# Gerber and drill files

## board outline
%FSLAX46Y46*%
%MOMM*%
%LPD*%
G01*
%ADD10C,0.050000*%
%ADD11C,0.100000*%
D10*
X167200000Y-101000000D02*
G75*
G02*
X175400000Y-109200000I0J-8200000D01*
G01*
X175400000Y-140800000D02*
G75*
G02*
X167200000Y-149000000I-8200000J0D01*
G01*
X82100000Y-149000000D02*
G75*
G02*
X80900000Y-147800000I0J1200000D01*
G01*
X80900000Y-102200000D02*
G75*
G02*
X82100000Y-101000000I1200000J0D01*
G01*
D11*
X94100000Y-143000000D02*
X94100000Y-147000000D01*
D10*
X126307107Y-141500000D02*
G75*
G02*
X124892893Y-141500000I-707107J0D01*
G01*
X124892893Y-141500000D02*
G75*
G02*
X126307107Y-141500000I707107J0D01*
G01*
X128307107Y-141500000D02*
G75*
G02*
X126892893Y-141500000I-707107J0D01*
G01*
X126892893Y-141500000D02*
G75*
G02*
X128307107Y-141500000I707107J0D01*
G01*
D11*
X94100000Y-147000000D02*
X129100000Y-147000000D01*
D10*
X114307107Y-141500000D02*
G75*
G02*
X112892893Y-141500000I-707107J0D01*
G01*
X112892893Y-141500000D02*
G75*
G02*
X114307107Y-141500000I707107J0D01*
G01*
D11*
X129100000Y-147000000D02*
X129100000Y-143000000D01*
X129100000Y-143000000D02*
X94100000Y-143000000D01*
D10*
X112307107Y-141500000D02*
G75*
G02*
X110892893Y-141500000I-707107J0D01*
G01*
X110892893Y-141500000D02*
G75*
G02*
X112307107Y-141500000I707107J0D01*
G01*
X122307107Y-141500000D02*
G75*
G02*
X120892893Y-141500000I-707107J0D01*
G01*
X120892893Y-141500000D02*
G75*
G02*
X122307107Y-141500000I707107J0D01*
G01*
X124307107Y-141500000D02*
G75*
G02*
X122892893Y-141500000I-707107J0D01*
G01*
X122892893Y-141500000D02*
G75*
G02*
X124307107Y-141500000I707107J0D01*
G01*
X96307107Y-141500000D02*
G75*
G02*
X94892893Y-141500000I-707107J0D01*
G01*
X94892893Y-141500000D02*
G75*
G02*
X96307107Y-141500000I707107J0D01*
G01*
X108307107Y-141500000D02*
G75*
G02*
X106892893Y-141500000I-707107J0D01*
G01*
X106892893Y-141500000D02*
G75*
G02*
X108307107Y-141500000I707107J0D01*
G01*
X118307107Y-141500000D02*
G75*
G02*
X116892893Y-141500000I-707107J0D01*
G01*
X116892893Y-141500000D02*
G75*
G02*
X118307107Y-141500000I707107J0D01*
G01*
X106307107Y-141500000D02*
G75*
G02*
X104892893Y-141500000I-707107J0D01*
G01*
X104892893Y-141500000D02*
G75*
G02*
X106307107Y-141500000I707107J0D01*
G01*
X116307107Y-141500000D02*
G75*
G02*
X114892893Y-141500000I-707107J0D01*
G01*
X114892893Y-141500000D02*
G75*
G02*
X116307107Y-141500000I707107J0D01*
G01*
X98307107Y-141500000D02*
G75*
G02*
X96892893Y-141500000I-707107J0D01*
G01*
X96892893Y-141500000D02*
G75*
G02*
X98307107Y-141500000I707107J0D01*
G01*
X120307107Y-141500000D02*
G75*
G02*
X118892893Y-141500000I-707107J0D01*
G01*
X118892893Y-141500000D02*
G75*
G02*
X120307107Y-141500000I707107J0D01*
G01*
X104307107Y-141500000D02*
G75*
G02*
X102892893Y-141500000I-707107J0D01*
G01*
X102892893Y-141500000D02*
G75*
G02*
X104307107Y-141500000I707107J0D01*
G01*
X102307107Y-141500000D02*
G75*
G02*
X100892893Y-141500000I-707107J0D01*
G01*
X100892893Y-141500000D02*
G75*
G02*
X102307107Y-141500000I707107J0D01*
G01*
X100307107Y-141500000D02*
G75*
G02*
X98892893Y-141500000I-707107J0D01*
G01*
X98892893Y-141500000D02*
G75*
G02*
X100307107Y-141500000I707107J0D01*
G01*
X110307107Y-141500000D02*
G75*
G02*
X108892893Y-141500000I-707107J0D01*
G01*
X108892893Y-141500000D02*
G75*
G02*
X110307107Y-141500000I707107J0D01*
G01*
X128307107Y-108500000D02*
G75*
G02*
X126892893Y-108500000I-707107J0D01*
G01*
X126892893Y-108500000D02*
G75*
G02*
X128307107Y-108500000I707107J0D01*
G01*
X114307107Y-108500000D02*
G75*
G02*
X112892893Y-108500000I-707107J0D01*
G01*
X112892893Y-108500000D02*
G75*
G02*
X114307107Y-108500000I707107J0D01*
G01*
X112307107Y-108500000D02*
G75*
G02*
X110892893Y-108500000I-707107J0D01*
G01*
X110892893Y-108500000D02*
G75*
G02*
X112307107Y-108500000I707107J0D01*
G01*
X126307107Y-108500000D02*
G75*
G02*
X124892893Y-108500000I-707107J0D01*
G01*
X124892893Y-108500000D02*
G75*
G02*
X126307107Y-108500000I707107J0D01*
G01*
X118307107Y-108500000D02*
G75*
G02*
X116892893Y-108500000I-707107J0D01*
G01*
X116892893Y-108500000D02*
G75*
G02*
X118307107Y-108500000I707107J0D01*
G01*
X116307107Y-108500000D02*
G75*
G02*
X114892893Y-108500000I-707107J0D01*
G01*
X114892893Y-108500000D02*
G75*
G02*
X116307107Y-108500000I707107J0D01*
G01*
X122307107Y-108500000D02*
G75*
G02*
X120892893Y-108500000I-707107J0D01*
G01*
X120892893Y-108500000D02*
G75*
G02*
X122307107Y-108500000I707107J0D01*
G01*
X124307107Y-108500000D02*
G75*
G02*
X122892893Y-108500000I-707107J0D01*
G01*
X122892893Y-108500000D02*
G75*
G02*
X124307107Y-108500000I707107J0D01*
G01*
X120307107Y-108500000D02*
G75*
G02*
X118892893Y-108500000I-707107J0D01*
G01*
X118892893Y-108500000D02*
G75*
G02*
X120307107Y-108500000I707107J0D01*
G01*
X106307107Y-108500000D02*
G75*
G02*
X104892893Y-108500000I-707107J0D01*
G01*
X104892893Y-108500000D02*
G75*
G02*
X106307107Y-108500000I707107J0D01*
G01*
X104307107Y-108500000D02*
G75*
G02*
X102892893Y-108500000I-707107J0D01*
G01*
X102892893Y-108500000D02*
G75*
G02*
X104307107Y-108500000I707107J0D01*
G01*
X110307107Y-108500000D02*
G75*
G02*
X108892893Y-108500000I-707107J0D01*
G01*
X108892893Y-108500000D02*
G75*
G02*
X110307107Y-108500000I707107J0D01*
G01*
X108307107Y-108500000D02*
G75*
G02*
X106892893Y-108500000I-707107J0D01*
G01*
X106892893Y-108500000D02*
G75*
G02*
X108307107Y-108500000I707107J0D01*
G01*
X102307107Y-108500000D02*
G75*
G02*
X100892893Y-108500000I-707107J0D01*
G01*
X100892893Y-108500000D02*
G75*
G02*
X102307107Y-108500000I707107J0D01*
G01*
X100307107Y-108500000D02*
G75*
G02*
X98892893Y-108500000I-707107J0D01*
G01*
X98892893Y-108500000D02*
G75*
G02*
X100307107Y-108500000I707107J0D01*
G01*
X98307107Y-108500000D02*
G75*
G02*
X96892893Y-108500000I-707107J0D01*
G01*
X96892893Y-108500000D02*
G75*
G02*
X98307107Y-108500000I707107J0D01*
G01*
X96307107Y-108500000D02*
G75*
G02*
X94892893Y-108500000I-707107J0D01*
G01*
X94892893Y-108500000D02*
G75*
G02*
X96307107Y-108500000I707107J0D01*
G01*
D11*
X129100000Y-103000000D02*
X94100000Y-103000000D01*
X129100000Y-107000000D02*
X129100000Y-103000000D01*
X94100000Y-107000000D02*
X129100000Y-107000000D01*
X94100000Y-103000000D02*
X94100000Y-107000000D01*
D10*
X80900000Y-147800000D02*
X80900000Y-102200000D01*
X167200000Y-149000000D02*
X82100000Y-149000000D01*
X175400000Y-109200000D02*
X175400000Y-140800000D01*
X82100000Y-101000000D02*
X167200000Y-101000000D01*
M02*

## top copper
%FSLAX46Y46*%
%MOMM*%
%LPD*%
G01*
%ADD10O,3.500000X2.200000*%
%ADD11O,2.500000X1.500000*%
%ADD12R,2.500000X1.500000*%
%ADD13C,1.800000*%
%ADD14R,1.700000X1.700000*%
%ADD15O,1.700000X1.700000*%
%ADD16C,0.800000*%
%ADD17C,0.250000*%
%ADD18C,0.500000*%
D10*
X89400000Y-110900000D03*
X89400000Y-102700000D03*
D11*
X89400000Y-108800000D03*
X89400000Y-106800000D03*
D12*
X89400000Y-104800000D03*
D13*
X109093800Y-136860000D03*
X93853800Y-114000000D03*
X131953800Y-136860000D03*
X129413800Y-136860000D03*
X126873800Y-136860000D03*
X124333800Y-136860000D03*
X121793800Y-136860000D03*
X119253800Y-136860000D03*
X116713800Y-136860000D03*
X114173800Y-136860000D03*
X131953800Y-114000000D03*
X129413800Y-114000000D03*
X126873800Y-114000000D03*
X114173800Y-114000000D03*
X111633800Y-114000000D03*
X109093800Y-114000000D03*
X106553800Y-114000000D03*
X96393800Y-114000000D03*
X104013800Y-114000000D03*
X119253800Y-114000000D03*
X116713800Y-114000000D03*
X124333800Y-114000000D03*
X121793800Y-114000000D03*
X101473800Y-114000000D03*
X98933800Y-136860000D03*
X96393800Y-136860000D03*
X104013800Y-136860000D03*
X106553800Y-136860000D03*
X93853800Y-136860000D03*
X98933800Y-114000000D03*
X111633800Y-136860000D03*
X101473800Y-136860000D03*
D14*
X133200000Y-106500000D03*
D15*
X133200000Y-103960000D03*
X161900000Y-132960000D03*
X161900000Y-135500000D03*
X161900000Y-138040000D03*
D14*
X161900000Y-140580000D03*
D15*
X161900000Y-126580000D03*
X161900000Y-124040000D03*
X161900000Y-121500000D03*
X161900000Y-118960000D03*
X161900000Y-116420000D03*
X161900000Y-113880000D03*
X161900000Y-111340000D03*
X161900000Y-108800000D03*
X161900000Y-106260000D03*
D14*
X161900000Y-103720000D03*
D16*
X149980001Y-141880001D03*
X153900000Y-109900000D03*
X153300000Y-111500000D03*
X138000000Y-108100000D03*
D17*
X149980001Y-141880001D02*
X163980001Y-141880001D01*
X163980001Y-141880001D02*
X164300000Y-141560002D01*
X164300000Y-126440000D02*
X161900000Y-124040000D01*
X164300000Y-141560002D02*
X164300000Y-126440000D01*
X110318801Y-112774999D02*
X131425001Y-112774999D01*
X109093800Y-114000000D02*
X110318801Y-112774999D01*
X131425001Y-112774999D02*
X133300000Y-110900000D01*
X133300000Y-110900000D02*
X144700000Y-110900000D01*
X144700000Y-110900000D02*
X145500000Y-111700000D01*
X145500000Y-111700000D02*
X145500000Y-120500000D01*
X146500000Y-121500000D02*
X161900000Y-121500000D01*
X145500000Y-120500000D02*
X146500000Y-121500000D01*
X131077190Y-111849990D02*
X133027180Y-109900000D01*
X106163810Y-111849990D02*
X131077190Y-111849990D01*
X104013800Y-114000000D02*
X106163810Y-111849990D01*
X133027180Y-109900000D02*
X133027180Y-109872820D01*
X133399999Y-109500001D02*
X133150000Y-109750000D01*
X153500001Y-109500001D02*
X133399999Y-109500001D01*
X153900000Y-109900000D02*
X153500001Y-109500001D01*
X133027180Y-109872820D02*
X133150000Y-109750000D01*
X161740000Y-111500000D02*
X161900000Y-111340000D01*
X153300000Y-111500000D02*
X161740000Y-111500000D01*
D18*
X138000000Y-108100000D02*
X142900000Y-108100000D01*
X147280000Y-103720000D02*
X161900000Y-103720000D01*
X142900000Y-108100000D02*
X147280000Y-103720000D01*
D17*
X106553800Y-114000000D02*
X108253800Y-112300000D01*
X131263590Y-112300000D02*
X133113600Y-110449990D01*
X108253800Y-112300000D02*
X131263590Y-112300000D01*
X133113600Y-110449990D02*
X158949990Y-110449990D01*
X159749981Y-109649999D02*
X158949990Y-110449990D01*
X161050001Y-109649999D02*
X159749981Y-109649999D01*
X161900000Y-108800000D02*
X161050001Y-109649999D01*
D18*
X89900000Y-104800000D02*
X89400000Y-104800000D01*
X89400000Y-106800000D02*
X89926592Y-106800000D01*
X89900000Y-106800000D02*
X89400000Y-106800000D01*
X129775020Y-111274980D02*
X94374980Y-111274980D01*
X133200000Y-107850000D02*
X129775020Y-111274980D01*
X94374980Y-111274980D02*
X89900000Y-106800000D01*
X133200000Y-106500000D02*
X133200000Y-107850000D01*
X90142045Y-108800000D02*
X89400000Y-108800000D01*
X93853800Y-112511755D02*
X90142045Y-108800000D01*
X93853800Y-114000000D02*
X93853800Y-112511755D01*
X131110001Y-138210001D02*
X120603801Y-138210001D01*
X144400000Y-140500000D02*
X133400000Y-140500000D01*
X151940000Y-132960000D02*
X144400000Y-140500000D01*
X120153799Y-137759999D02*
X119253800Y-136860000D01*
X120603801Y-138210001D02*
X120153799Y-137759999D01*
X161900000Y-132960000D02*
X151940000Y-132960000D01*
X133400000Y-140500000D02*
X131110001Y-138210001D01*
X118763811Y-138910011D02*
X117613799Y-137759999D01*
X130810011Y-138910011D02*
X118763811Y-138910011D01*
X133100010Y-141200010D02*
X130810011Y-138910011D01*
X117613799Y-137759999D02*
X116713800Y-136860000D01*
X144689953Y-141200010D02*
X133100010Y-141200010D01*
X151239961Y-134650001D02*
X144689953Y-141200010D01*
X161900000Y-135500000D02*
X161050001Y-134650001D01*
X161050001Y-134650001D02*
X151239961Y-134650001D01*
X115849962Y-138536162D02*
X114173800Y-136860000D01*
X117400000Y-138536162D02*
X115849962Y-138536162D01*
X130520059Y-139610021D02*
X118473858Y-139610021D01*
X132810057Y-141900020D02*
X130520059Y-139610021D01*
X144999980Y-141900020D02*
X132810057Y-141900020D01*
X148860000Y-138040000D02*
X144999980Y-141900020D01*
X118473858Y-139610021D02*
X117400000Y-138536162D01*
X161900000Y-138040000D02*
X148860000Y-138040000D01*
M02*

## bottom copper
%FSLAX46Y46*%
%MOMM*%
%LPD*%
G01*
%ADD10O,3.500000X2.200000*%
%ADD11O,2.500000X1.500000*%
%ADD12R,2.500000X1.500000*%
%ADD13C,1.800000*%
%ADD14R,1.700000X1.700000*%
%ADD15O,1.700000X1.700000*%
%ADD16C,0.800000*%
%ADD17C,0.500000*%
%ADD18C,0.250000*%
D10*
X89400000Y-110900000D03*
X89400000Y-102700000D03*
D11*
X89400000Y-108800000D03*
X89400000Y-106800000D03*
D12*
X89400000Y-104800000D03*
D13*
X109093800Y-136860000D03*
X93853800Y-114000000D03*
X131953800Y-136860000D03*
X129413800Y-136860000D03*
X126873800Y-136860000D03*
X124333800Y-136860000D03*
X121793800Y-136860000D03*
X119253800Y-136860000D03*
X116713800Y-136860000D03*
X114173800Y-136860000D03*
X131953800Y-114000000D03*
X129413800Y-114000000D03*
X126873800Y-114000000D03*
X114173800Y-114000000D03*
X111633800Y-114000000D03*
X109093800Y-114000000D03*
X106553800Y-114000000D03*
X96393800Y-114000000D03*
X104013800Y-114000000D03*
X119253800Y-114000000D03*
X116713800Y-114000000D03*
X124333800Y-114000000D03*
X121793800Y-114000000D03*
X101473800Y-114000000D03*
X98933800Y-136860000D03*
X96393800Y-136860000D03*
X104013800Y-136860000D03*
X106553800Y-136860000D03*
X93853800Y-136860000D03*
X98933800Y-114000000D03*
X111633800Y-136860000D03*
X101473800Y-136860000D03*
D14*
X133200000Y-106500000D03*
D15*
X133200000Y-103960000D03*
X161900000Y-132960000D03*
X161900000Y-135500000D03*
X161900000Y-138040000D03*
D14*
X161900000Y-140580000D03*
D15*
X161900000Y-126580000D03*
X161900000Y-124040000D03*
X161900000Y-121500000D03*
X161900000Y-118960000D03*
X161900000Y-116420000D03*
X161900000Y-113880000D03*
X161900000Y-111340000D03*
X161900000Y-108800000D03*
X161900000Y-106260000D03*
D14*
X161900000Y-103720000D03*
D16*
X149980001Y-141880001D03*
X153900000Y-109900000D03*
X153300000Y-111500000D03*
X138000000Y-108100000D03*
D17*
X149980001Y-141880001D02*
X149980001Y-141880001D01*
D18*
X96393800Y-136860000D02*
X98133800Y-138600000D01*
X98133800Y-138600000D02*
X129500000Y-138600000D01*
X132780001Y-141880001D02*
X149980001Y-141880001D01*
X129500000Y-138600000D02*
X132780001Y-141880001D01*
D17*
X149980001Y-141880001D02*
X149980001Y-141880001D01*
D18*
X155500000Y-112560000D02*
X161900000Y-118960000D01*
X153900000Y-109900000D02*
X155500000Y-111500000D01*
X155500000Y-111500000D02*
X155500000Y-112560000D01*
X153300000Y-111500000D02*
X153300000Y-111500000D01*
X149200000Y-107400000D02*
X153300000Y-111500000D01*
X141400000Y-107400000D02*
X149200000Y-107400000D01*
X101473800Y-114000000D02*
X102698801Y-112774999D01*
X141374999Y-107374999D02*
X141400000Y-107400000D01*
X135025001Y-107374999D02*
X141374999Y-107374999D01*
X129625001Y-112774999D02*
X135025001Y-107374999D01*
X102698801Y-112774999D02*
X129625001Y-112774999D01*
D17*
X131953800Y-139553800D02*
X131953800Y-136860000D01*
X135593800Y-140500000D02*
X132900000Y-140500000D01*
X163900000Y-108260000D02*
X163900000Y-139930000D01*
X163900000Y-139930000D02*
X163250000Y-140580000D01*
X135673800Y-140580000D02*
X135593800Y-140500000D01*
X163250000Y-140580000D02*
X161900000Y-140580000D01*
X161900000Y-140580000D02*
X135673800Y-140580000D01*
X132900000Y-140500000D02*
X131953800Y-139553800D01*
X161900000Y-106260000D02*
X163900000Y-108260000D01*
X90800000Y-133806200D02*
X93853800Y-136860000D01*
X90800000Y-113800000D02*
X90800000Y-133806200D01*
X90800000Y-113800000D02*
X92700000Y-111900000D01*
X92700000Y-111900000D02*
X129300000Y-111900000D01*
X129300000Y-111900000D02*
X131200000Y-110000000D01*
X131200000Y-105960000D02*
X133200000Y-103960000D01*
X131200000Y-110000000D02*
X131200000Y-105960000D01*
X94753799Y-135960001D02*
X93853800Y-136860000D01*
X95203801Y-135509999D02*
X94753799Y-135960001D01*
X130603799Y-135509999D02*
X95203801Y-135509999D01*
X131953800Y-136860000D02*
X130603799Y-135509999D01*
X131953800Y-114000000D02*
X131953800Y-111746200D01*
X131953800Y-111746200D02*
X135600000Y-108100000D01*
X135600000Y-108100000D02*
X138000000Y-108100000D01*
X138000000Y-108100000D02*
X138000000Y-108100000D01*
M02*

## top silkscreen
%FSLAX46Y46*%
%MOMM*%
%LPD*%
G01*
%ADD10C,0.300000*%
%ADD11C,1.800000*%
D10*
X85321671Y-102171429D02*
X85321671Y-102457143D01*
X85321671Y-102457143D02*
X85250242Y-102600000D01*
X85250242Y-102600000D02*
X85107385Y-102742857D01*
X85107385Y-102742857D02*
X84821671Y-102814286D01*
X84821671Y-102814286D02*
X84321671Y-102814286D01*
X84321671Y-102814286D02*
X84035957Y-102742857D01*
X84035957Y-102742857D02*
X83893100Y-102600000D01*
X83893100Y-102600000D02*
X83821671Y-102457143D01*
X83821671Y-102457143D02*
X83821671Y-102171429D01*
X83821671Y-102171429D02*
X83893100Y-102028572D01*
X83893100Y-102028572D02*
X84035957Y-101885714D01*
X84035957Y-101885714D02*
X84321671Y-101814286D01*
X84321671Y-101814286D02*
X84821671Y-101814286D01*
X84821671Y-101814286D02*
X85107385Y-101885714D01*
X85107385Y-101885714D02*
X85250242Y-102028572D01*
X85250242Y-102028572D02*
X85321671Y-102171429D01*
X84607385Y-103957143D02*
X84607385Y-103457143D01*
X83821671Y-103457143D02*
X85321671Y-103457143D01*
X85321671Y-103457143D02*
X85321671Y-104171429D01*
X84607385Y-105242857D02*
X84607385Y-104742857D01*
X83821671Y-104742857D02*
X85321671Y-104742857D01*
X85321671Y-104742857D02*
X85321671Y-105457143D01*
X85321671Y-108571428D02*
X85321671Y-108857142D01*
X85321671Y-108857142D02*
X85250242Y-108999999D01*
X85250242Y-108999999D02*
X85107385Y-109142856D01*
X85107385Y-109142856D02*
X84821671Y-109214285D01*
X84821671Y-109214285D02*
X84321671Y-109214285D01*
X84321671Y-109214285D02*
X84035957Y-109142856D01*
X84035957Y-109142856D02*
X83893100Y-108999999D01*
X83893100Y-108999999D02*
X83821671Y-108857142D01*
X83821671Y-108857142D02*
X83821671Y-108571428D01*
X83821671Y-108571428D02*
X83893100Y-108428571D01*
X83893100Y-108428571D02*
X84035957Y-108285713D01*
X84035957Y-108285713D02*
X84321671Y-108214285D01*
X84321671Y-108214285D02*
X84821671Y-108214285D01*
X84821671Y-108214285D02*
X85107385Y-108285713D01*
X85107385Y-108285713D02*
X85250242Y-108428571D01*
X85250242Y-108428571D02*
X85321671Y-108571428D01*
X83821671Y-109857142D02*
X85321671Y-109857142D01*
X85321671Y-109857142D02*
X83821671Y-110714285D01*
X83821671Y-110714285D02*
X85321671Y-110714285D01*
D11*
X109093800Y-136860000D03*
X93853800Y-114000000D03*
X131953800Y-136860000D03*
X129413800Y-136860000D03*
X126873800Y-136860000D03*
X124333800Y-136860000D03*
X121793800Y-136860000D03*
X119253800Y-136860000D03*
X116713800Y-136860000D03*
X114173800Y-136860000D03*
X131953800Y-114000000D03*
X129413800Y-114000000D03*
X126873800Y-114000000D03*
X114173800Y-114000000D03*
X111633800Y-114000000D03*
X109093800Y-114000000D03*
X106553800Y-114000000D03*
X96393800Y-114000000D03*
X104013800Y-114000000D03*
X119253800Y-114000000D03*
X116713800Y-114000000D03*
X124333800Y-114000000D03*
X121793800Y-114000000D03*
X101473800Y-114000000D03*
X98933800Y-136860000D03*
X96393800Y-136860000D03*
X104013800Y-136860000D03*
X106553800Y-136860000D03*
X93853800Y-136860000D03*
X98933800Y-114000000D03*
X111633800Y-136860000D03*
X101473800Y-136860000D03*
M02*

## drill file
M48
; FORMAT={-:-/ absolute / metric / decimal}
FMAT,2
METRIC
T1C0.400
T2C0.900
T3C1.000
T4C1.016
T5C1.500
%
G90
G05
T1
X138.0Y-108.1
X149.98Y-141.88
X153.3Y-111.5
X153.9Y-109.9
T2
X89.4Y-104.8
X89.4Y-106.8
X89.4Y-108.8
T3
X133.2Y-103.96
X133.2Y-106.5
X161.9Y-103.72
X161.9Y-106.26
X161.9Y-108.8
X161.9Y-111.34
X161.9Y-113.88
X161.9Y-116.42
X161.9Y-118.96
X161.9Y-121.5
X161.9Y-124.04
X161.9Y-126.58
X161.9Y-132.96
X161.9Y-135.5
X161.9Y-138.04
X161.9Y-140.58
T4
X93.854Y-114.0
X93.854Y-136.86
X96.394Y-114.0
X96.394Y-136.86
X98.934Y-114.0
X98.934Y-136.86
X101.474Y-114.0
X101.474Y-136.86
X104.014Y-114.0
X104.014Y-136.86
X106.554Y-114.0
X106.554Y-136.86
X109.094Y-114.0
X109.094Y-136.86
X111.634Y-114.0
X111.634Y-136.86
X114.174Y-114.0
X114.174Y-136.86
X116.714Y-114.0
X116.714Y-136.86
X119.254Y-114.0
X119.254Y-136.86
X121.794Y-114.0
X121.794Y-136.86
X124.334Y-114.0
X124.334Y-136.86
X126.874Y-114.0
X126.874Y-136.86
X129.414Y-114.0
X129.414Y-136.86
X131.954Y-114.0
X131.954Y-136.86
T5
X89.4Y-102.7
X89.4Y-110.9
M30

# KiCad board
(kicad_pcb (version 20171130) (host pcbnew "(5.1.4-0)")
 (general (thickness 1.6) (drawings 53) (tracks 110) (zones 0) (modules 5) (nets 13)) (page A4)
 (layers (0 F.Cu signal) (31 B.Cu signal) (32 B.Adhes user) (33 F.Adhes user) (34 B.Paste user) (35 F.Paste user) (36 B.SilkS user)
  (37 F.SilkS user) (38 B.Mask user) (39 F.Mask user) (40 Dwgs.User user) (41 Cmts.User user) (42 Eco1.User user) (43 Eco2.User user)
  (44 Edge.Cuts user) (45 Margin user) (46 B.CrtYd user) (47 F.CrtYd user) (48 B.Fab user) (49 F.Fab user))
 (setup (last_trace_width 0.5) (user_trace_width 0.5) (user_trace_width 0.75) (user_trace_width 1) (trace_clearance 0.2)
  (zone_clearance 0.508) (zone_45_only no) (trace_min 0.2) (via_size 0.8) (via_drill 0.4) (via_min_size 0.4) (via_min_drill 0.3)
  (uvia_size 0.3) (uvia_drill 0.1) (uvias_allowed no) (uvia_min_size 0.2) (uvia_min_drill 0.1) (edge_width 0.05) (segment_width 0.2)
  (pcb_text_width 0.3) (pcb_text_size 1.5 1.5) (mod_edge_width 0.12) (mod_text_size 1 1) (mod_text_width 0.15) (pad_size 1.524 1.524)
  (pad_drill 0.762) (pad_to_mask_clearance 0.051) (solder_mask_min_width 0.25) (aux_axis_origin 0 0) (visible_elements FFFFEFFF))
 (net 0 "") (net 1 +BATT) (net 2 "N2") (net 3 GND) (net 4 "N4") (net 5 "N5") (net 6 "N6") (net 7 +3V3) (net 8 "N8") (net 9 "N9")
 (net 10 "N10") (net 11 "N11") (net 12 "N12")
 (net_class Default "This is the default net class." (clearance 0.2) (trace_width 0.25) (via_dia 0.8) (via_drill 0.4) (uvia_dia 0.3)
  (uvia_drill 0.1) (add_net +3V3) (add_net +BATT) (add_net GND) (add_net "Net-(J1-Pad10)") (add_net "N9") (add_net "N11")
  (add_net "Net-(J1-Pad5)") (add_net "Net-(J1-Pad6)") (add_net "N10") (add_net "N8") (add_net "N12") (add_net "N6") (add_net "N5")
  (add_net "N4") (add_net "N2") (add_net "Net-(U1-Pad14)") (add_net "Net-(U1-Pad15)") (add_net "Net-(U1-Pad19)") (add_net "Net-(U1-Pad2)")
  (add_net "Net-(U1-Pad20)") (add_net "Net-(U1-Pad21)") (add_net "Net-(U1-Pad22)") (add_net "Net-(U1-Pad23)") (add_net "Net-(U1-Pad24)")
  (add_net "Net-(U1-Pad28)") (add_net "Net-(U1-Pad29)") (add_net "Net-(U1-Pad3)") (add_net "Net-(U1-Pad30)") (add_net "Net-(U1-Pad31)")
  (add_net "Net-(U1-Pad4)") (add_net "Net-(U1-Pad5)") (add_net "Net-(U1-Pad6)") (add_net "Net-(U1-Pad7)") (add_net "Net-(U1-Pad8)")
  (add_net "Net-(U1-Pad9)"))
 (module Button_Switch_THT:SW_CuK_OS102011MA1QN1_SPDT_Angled (layer F.Cu) (at 89.4 104.8 270)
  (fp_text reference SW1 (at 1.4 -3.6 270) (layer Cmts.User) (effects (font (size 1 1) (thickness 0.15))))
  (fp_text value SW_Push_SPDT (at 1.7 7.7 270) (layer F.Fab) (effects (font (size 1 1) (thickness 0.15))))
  (pad "" thru_hole oval (at 6.1 0 270) (size 2.2 3.5) (drill 1.5) (layers *.Cu *.Mask))
  (pad "" thru_hole oval (at -2.1 0 270) (size 2.2 3.5) (drill 1.5) (layers *.Cu *.Mask))
  (pad 3 thru_hole oval (at 4 0 270) (size 1.5 2.5) (drill 0.9) (layers *.Cu *.Mask) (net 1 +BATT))
  (pad 2 thru_hole oval (at 2 0 270) (size 1.5 2.5) (drill 0.9) (layers *.Cu *.Mask) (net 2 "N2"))
  (pad 1 thru_hole rect (at 0 0 270) (size 1.5 2.5) (drill 0.9) (layers *.Cu *.Mask)))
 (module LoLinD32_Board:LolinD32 (layer F.Cu) (at 107.9 125.7094 270)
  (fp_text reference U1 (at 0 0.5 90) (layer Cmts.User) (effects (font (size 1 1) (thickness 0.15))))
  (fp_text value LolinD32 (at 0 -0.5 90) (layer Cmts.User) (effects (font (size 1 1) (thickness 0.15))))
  (pad 23 thru_hole circle (at 11.1506 -1.1938 270) (size 1.8 1.8) (drill 1.016) (layers *.Cu *.Mask F.SilkS))
  (pad 16 thru_hole circle (at -11.7094 14.0462 270) (size 1.8 1.8) (drill 1.016) (layers *.Cu *.Mask F.SilkS) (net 1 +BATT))
  (pad 32 thru_hole circle (at 11.1506 -24.0538 270) (size 1.8 1.8) (drill 1.016) (layers *.Cu *.Mask F.SilkS) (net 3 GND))
  (pad 31 thru_hole circle (at 11.1506 -21.5138 270) (size 1.8 1.8) (drill 1.016) (layers *.Cu *.Mask F.SilkS))
  (pad 30 thru_hole circle (at 11.1506 -18.9738 270) (size 1.8 1.8) (drill 1.016) (layers *.Cu *.Mask F.SilkS))
  (pad 29 thru_hole circle (at 11.1506 -16.4338 270) (size 1.8 1.8) (drill 1.016) (layers *.Cu *.Mask F.SilkS))
  (pad 28 thru_hole circle (at 11.1506 -13.8938 270) (size 1.8 1.8) (drill 1.016) (layers *.Cu *.Mask F.SilkS))
  (pad 27 thru_hole circle (at 11.1506 -11.3538 270) (size 1.8 1.8) (drill 1.016) (layers *.Cu *.Mask F.SilkS) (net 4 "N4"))
  (pad 26 thru_hole circle (at 11.1506 -8.8138 270) (size 1.8 1.8) (drill 1.016) (layers *.Cu *.Mask F.SilkS) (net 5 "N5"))
  (pad 25 thru_hole circle (at 11.1506 -6.2738 270) (size 1.8 1.8) (drill 1.016) (layers *.Cu *.Mask F.SilkS) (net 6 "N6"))
  (pad 1 thru_hole circle (at -11.7094 -24.0538 270) (size 1.8 1.8) (drill 1.016) (layers *.Cu *.Mask F.SilkS) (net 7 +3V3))
  (pad 2 thru_hole circle (at -11.7094 -21.5138 270) (size 1.8 1.8) (drill 1.016) (layers *.Cu *.Mask F.SilkS))
  (pad 3 thru_hole circle (at -11.7094 -18.9738 270) (size 1.8 1.8) (drill 1.016) (layers *.Cu *.Mask F.SilkS))
  (pad 8 thru_hole circle (at -11.7094 -6.2738 270) (size 1.8 1.8) (drill 1.016) (layers *.Cu *.Mask F.SilkS))
  (pad 9 thru_hole circle (at -11.7094 -3.7338 270) (size 1.8 1.8) (drill 1.016) (layers *.Cu *.Mask F.SilkS))
  (pad 10 thru_hole circle (at -11.7094 -1.1938 270) (size 1.8 1.8) (drill 1.016) (layers *.Cu *.Mask F.SilkS) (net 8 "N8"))
  (pad 11 thru_hole circle (at -11.7094 1.3462 270) (size 1.8 1.8) (drill 1.016) (layers *.Cu *.Mask F.SilkS) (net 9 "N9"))
  (pad 15 thru_hole circle (at -11.7094 11.5062 270) (size 1.8 1.8) (drill 1.016) (layers *.Cu *.Mask F.SilkS))
  (pad 12 thru_hole circle (at -11.7094 3.8862 270) (size 1.8 1.8) (drill 1.016) (layers *.Cu *.Mask F.SilkS) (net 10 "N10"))
  (pad 6 thru_hole circle (at -11.7094 -11.3538 270) (size 1.8 1.8) (drill 1.016) (layers *.Cu *.Mask F.SilkS))
  (pad 7 thru_hole circle (at -11.7094 -8.8138 270) (size 1.8 1.8) (drill 1.016) (layers *.Cu *.Mask F.SilkS))
  (pad 4 thru_hole circle (at -11.7094 -16.4338 270) (size 1.8 1.8) (drill 1.016) (layers *.Cu *.Mask F.SilkS))
  (pad 5 thru_hole circle (at -11.7094 -13.8938 270) (size 1.8 1.8) (drill 1.016) (layers *.Cu *.Mask F.SilkS))
  (pad 13 thru_hole circle (at -11.7094 6.4262 270) (size 1.8 1.8) (drill 1.016) (layers *.Cu *.Mask F.SilkS) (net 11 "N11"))
  (pad 19 thru_hole circle (at 11.1506 8.9662 270) (size 1.8 1.8) (drill 1.016) (layers *.Cu *.Mask F.SilkS))
  (pad 18 thru_hole circle (at 11.1506 11.5062 270) (size 1.8 1.8) (drill 1.016) (layers *.Cu *.Mask F.SilkS) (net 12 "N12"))
  (pad 21 thru_hole circle (at 11.1506 3.8862 270) (size 1.8 1.8) (drill 1.016) (layers *.Cu *.Mask F.SilkS))
  (pad 22 thru_hole circle (at 11.1506 1.3462 270) (size 1.8 1.8) (drill 1.016) (layers *.Cu *.Mask F.SilkS))
  (pad 17 thru_hole circle (at 11.1506 14.0462 270) (size 1.8 1.8) (drill 1.016) (layers *.Cu *.Mask F.SilkS) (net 3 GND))
  (pad 14 thru_hole circle (at -11.7094 8.9662 270) (size 1.8 1.8) (drill 1.016) (layers *.Cu *.Mask F.SilkS))
  (pad 24 thru_hole circle (at 11.1506 -3.7338 270) (size 1.8 1.8) (drill 1.016) (layers *.Cu *.Mask F.SilkS))
  (pad 20 thru_hole circle (at 11.1506 6.4262 270) (size 1.8 1.8) (drill 1.016) (layers *.Cu *.Mask F.SilkS)))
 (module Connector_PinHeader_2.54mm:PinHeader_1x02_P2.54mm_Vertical (layer F.Cu) (at 133.2 106.5 180)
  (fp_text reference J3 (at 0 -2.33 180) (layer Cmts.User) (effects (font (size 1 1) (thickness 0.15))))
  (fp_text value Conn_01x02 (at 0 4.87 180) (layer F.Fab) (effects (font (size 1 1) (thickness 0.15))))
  (pad 1 thru_hole rect (at 0 0 180) (size 1.7 1.7) (drill 1) (layers *.Cu *.Mask) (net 2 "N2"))
  (pad 2 thru_hole oval (at 0 2.54 180) (size 1.7 1.7) (drill 1) (layers *.Cu *.Mask) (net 3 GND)))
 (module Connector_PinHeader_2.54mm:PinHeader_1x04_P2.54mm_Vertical (layer F.Cu) (at 161.9 140.58 180)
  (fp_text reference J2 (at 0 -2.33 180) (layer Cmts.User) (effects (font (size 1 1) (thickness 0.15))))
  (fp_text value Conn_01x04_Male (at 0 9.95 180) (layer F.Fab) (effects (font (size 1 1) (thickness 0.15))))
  (pad 4 thru_hole oval (at 0 7.62 180) (size 1.7 1.7) (drill 1) (layers *.Cu *.Mask) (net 4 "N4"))
  (pad 3 thru_hole oval (at 0 5.08 180) (size 1.7 1.7) (drill 1) (layers *.Cu *.Mask) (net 5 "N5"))
  (pad 2 thru_hole oval (at 0 2.54 180) (size 1.7 1.7) (drill 1) (layers *.Cu *.Mask) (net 6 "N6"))
  (pad 1 thru_hole rect (at 0 0 180) (size 1.7 1.7) (drill 1) (layers *.Cu *.Mask) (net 3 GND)))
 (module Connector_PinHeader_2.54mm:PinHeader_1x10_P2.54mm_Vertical (layer F.Cu) (at 161.9 103.72)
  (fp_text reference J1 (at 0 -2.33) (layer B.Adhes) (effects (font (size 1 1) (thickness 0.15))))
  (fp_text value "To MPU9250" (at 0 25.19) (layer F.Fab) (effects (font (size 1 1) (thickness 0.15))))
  (pad 10 thru_hole oval (at 0 22.86) (size 1.7 1.7) (drill 1) (layers *.Cu *.Mask))
  (pad 9 thru_hole oval (at 0 20.32) (size 1.7 1.7) (drill 1) (layers *.Cu *.Mask) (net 12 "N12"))
  (pad 8 thru_hole oval (at 0 17.78) (size 1.7 1.7) (drill 1) (layers *.Cu *.Mask) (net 8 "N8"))
  (pad 7 thru_hole oval (at 0 15.24) (size 1.7 1.7) (drill 1) (layers *.Cu *.Mask) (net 10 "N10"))
  (pad 6 thru_hole oval (at 0 12.7) (size 1.7 1.7) (drill 1) (layers *.Cu *.Mask))
  (pad 5 thru_hole oval (at 0 10.16) (size 1.7 1.7) (drill 1) (layers *.Cu *.Mask))
  (pad 4 thru_hole oval (at 0 7.62) (size 1.7 1.7) (drill 1) (layers *.Cu *.Mask) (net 11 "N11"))
  (pad 3 thru_hole oval (at 0 5.08) (size 1.7 1.7) (drill 1) (layers *.Cu *.Mask) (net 9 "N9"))
  (pad 2 thru_hole oval (at 0 2.54) (size 1.7 1.7) (drill 1) (layers *.Cu *.Mask) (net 3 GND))
  (pad 1 thru_hole rect (at 0 0) (size 1.7 1.7) (drill 1) (layers *.Cu *.Mask) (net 7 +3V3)))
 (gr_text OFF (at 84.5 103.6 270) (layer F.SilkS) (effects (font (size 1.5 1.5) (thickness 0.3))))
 (gr_arc (start 167.2 109.2) (end 175.4 109.2) (angle -90) (layer Edge.Cuts) (width 0.05))
 (gr_arc (start 167.2 140.8) (end 167.2 149) (angle -90) (layer Edge.Cuts) (width 0.05))
 (gr_arc (start 82.1 147.8) (end 80.9 147.8) (angle -90) (layer Edge.Cuts) (width 0.05))
 (gr_arc (start 82.1 102.2) (end 82.1 101) (angle -90) (layer Edge.Cuts) (width 0.05))
 (gr_line (start 94.1 143) (end 94.1 147) (layer Edge.Cuts) (width 0.1))
 (gr_circle (center 125.6 141.5) (end 125.1 141) (layer Edge.Cuts) (width 0.05))
 (gr_circle (center 127.6 141.5) (end 127.1 141) (layer Edge.Cuts) (width 0.05))
 (gr_line (start 94.1 147) (end 129.1 147) (layer Edge.Cuts) (width 0.1))
 (gr_circle (center 113.6 141.5) (end 113.1 141) (layer Edge.Cuts) (width 0.05))
 (gr_line (start 129.1 147) (end 129.1 143) (layer Edge.Cuts) (width 0.1))
 (gr_line (start 129.1 143) (end 94.1 143) (layer Edge.Cuts) (width 0.1))
 (gr_circle (center 111.6 141.5) (end 111.1 141) (layer Edge.Cuts) (width 0.05))
 (gr_circle (center 121.6 141.5) (end 121.1 141) (layer Edge.Cuts) (width 0.05))
 (gr_circle (center 123.6 141.5) (end 123.1 141) (layer Edge.Cuts) (width 0.05))
 (gr_circle (center 95.6 141.5) (end 95.1 141) (layer Edge.Cuts) (width 0.05))
 (gr_circle (center 107.6 141.5) (end 107.1 141) (layer Edge.Cuts) (width 0.05))
 (gr_circle (center 117.6 141.5) (end 117.1 141) (layer Edge.Cuts) (width 0.05))
 (gr_circle (center 105.6 141.5) (end 105.1 141) (layer Edge.Cuts) (width 0.05))
 (gr_circle (center 115.6 141.5) (end 115.1 141) (layer Edge.Cuts) (width 0.05))
 (gr_circle (center 97.6 141.5) (end 97.1 141) (layer Edge.Cuts) (width 0.05))
 (gr_circle (center 119.6 141.5) (end 119.1 141) (layer Edge.Cuts) (width 0.05))
 (gr_circle (center 103.6 141.5) (end 103.1 141) (layer Edge.Cuts) (width 0.05))
 (gr_circle (center 101.6 141.5) (end 101.1 141) (layer Edge.Cuts) (width 0.05))
 (gr_circle (center 99.6 141.5) (end 99.1 141) (layer Edge.Cuts) (width 0.05))
 (gr_circle (center 109.6 141.5) (end 109.1 141) (layer Edge.Cuts) (width 0.05))
 (gr_circle (center 127.6 108.5) (end 128.1 109) (layer Edge.Cuts) (width 0.05))
 (gr_circle (center 113.6 108.5) (end 114.1 109) (layer Edge.Cuts) (width 0.05))
 (gr_circle (center 111.6 108.5) (end 112.1 109) (layer Edge.Cuts) (width 0.05))
 (gr_circle (center 125.6 108.5) (end 126.1 109) (layer Edge.Cuts) (width 0.05))
 (gr_circle (center 117.6 108.5) (end 118.1 109) (layer Edge.Cuts) (width 0.05))
 (gr_circle (center 115.6 108.5) (end 116.1 109) (layer Edge.Cuts) (width 0.05))
 (gr_circle (center 121.6 108.5) (end 122.1 109) (layer Edge.Cuts) (width 0.05))
 (gr_circle (center 123.6 108.5) (end 124.1 109) (layer Edge.Cuts) (width 0.05))
 (gr_circle (center 119.6 108.5) (end 120.1 109) (layer Edge.Cuts) (width 0.05))
 (gr_circle (center 105.6 108.5) (end 106.1 109) (layer Edge.Cuts) (width 0.05))
 (gr_circle (center 103.6 108.5) (end 104.1 109) (layer Edge.Cuts) (width 0.05))
 (gr_circle (center 109.6 108.5) (end 110.1 109) (layer Edge.Cuts) (width 0.05))
 (gr_circle (center 107.6 108.5) (end 108.1 109) (layer Edge.Cuts) (width 0.05))
 (gr_circle (center 101.6 108.5) (end 102.1 109) (layer Edge.Cuts) (width 0.05))
 (gr_circle (center 99.6 108.5) (end 100.1 109) (layer Edge.Cuts) (width 0.05))
 (gr_circle (center 97.6 108.5) (end 98.1 109) (layer Edge.Cuts) (width 0.05))
 (gr_circle (center 95.6 108.5) (end 96.1 109) (layer Edge.Cuts) (width 0.05))
 (gr_line (start 129.1 103) (end 94.1 103) (layer Edge.Cuts) (width 0.1))
 (gr_line (start 129.1 107) (end 129.1 103) (layer Edge.Cuts) (width 0.1))
 (gr_line (start 94.1 107) (end 129.1 107) (layer Edge.Cuts) (width 0.1))
 (gr_line (start 94.1 103) (end 94.1 107) (layer Edge.Cuts) (width 0.1))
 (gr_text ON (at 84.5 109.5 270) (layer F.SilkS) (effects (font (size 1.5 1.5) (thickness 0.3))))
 (gr_line (start 80.9 147.8) (end 80.9 102.2) (layer Edge.Cuts) (width 0.05))
 (gr_line (start 167.2 149) (end 82.1 149) (layer Edge.Cuts) (width 0.05))
 (gr_line (start 175.4 109.2) (end 175.4 140.8) (layer Edge.Cuts) (width 0.05))
 (gr_line (start 82.1 101) (end 167.2 101) (layer Edge.Cuts) (width 0.05))
 (segment (start 149.980001 141.880001) (end 149.980001 141.880001) (width 0.5) (layer B.Cu) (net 12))
 (segment (start 96.3938 136.86) (end 98.1338 138.6) (width 0.25) (layer B.Cu) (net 12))
 (segment (start 98.1338 138.6) (end 129.5 138.6) (width 0.25) (layer B.Cu) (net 12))
 (segment (start 132.780001 141.880001) (end 149.980001 141.880001) (width 0.25) (layer B.Cu) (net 12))
 (segment (start 129.5 138.6) (end 132.780001 141.880001) (width 0.25) (layer B.Cu) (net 12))
 (segment (start 149.980001 141.880001) (end 149.980001 141.880001) (width 0.5) (layer B.Cu) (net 12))
 (via (at 149.980001 141.880001) (size 0.8) (drill 0.4) (layers F.Cu B.Cu) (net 12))
 (segment (start 149.980001 141.880001) (end 163.980001 141.880001) (width 0.25) (layer F.Cu) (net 12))
 (segment (start 163.980001 141.880001) (end 164.3 141.560002) (width 0.25) (layer F.Cu) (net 12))
 (segment (start 164.3 126.44) (end 161.9 124.04) (width 0.25) (layer F.Cu) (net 12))
 (segment (start 164.3 141.560002) (end 164.3 126.44) (width 0.25) (layer F.Cu) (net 12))
 (segment (start 110.318801 112.774999) (end 131.425001 112.774999) (width 0.25) (layer F.Cu) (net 8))
 (segment (start 109.0938 114) (end 110.318801 112.774999) (width 0.25) (layer F.Cu) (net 8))
 (segment (start 131.425001 112.774999) (end 133.3 110.9) (width 0.25) (layer F.Cu) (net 8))
 (segment (start 133.3 110.9) (end 144.7 110.9) (width 0.25) (layer F.Cu) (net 8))
 (segment (start 144.7 110.9) (end 145.5 111.7) (width 0.25) (layer F.Cu) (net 8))
 (segment (start 145.5 111.7) (end 145.5 120.5) (width 0.25) (layer F.Cu) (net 8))
 (segment (start 146.5 121.5) (end 161.9 121.5) (width 0.25) (layer F.Cu) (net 8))
 (segment (start 145.5 120.5) (end 146.5 121.5) (width 0.25) (layer F.Cu) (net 8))
 (segment (start 131.07719 111.84999) (end 133.02718 109.9) (width 0.25) (layer F.Cu) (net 10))
 (segment (start 106.16381 111.84999) (end 131.07719 111.84999) (width 0.25) (layer F.Cu) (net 10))
 (segment (start 104.0138 114) (end 106.16381 111.84999) (width 0.25) (layer F.Cu) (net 10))
 (segment (start 133.02718 109.9) (end 133.02718 109.87282) (width 0.25) (layer F.Cu) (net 10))
 (via (at 153.9 109.9) (size 0.8) (drill 0.4) (layers F.Cu B.Cu) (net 10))
 (segment (start 155.5 112.56) (end 161.9 118.96) (width 0.25) (layer B.Cu) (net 10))
 (segment (start 153.9 109.9) (end 155.5 111.5) (width 0.25) (layer B.Cu) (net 10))
 (segment (start 155.5 111.5) (end 155.5 112.56) (width 0.25) (layer B.Cu) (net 10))
 (segment (start 133.399999 109.500001) (end 133.15 109.75) (width 0.25) (layer F.Cu) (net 10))
 (segment (start 153.500001 109.500001) (end 133.399999 109.500001) (width 0.25) (layer F.Cu) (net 10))
 (segment (start 153.9 109.9) (end 153.500001 109.500001) (width 0.25) (layer F.Cu) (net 10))
 (segment (start 133.02718 109.87282) (end 133.15 109.75) (width 0.25) (layer F.Cu) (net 10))
 (segment (start 153.3 111.5) (end 153.3 111.5) (width 0.25) (layer B.Cu) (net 11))
 (via (at 153.3 111.5) (size 0.8) (drill 0.4) (layers F.Cu B.Cu) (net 11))
 (segment (start 161.74 111.5) (end 161.9 111.34) (width 0.25) (layer F.Cu) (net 11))
 (segment (start 153.3 111.5) (end 161.74 111.5) (width 0.25) (layer F.Cu) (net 11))
 (segment (start 149.2 107.4) (end 153.3 111.5) (width 0.25) (layer B.Cu) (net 11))
 (segment (start 141.4 107.4) (end 149.2 107.4) (width 0.25) (layer B.Cu) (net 11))
 (segment (start 101.4738 114) (end 102.698801 112.774999) (width 0.25) (layer B.Cu) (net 11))
 (segment (start 141.374999 107.374999) (end 141.4 107.4) (width 0.25) (layer B.Cu) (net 11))
 (segment (start 135.025001 107.374999) (end 141.374999 107.374999) (width 0.25) (layer B.Cu) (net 11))
 (segment (start 129.625001 112.774999) (end 135.025001 107.374999) (width 0.25) (layer B.Cu) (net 11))
 (segment (start 102.698801 112.774999) (end 129.625001 112.774999) (width 0.25) (layer B.Cu) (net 11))
 (segment (start 131.9538 139.5538) (end 131.9538 136.86) (width 0.5) (layer B.Cu) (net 3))
 (segment (start 135.5938 140.5) (end 132.9 140.5) (width 0.5) (layer B.Cu) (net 3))
 (segment (start 163.9 108.26) (end 163.9 139.93) (width 0.5) (layer B.Cu) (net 3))
 (segment (start 163.9 139.93) (end 163.25 140.58) (width 0.5) (layer B.Cu) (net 3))
 (segment (start 135.6738 140.58) (end 135.5938 140.5) (width 0.5) (layer B.Cu) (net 3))
 (segment (start 163.25 140.58) (end 161.9 140.58) (width 0.5) (layer B.Cu) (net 3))
 (segment (start 161.9 140.58) (end 135.6738 140.58) (width 0.5) (layer B.Cu) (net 3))
 (segment (start 132.9 140.5) (end 131.9538 139.5538) (width 0.5) (layer B.Cu) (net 3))
 (segment (start 161.9 106.26) (end 163.9 108.26) (width 0.5) (layer B.Cu) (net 3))
 (segment (start 90.8 133.8062) (end 93.8538 136.86) (width 0.5) (layer B.Cu) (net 3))
 (segment (start 90.8 113.8) (end 90.8 133.8062) (width 0.5) (layer B.Cu) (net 3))
 (segment (start 90.8 113.8) (end 92.7 111.9) (width 0.5) (layer B.Cu) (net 3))
 (segment (start 92.7 111.9) (end 129.3 111.9) (width 0.5) (layer B.Cu) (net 3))
 (segment (start 129.3 111.9) (end 131.2 110) (width 0.5) (layer B.Cu) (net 3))
 (segment (start 131.2 105.96) (end 133.2 103.96) (width 0.5) (layer B.Cu) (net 3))
 (segment (start 131.2 110) (end 131.2 105.96) (width 0.5) (layer B.Cu) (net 3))
 (segment (start 94.753799 135.960001) (end 93.8538 136.86) (width 0.5) (layer B.Cu) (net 3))
 (segment (start 95.203801 135.509999) (end 94.753799 135.960001) (width 0.5) (layer B.Cu) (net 3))
 (segment (start 130.603799 135.509999) (end 95.203801 135.509999) (width 0.5) (layer B.Cu) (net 3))
 (segment (start 131.9538 136.86) (end 130.603799 135.509999) (width 0.5) (layer B.Cu) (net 3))
 (segment (start 131.9538 114) (end 131.9538 111.7462) (width 0.5) (layer B.Cu) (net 7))
 (segment (start 131.9538 111.7462) (end 135.6 108.1) (width 0.5) (layer B.Cu) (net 7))
 (segment (start 135.6 108.1) (end 138 108.1) (width 0.5) (layer B.Cu) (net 7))
 (segment (start 138 108.1) (end 138 108.1) (width 0.5) (layer B.Cu) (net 7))
 (via (at 138 108.1) (size 0.8) (drill 0.4) (layers F.Cu B.Cu) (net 7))
 (segment (start 138 108.1) (end 142.9 108.1) (width 0.5) (layer F.Cu) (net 7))
 (segment (start 147.28 103.72) (end 161.9 103.72) (width 0.5) (layer F.Cu) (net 7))
 (segment (start 142.9 108.1) (end 147.28 103.72) (width 0.5) (layer F.Cu) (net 7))
 (segment (start 106.5538 114) (end 108.2538 112.3) (width 0.25) (layer F.Cu) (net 9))
 (segment (start 131.26359 112.3) (end 133.1136 110.44999) (width 0.25) (layer F.Cu) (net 9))
 (segment (start 108.2538 112.3) (end 131.26359 112.3) (width 0.25) (layer F.Cu) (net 9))
 (segment (start 133.1136 110.44999) (end 158.94999 110.44999) (width 0.25) (layer F.Cu) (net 9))
 (segment (start 159.749981 109.649999) (end 158.94999 110.44999) (width 0.25) (layer F.Cu) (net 9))
 (segment (start 161.050001 109.649999) (end 159.749981 109.649999) (width 0.25) (layer F.Cu) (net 9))
 (segment (start 161.9 108.8) (end 161.050001 109.649999) (width 0.25) (layer F.Cu) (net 9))
 (segment (start 89.9 104.8) (end 89.4 104.8) (width 0.5) (layer F.Cu) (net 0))
 (segment (start 89.4 106.8) (end 89.926592 106.8) (width 0.5) (layer F.Cu) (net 2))
 (segment (start 89.9 106.8) (end 89.4 106.8) (width 0.5) (layer F.Cu) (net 2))
 (segment (start 129.77502 111.27498) (end 94.37498 111.27498) (width 0.5) (layer F.Cu) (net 2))
 (segment (start 133.2 107.85) (end 129.77502 111.27498) (width 0.5) (layer F.Cu) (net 2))
 (segment (start 94.37498 111.27498) (end 89.9 106.8) (width 0.5) (layer F.Cu) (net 2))
 (segment (start 133.2 106.5) (end 133.2 107.85) (width 0.5) (layer F.Cu) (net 2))
 (segment (start 90.142045 108.8) (end 89.4 108.8) (width 0.5) (layer F.Cu) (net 1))
 (segment (start 93.8538 112.511755) (end 90.142045 108.8) (width 0.5) (layer F.Cu) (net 1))
 (segment (start 93.8538 114) (end 93.8538 112.511755) (width 0.5) (layer F.Cu) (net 1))
 (segment (start 131.110001 138.210001) (end 120.603801 138.210001) (width 0.5) (layer F.Cu) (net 4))
 (segment (start 144.4 140.5) (end 133.4 140.5) (width 0.5) (layer F.Cu) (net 4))
 (segment (start 151.94 132.96) (end 144.4 140.5) (width 0.5) (layer F.Cu) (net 4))
 (segment (start 120.153799 137.759999) (end 119.2538 136.86) (width 0.5) (layer F.Cu) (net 4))
 (segment (start 120.603801 138.210001) (end 120.153799 137.759999) (width 0.5) (layer F.Cu) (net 4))
 (segment (start 161.9 132.96) (end 151.94 132.96) (width 0.5) (layer F.Cu) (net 4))
 (segment (start 133.4 140.5) (end 131.110001 138.210001) (width 0.5) (layer F.Cu) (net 4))
 (segment (start 118.763811 138.910011) (end 117.613799 137.759999) (width 0.5) (layer F.Cu) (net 5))
 (segment (start 130.810011 138.910011) (end 118.763811 138.910011) (width 0.5) (layer F.Cu) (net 5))
 (segment (start 133.10001 141.20001) (end 130.810011 138.910011) (width 0.5) (layer F.Cu) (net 5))
 (segment (start 117.613799 137.759999) (end 116.7138 136.86) (width 0.5) (layer F.Cu) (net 5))
 (segment (start 144.689953 141.20001) (end 133.10001 141.20001) (width 0.5) (layer F.Cu) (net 5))
 (segment (start 151.239961 134.650001) (end 144.689953 141.20001) (width 0.5) (layer F.Cu) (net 5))
 (segment (start 161.9 135.5) (end 161.050001 134.650001) (width 0.5) (layer F.Cu) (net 5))
 (segment (start 161.050001 134.650001) (end 151.239961 134.650001) (width 0.5) (layer F.Cu) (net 5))
 (segment (start 115.849962 138.536162) (end 114.1738 136.86) (width 0.5) (layer F.Cu) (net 6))
 (segment (start 117.4 138.536162) (end 115.849962 138.536162) (width 0.5) (layer F.Cu) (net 6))
 (segment (start 130.520059 139.610021) (end 118.473858 139.610021) (width 0.5) (layer F.Cu) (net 6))
 (segment (start 132.810057 141.90002) (end 130.520059 139.610021) (width 0.5) (layer F.Cu) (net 6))
 (segment (start 144.99998 141.90002) (end 132.810057 141.90002) (width 0.5) (layer F.Cu) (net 6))
 (segment (start 148.86 138.04) (end 144.99998 141.90002) (width 0.5) (layer F.Cu) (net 6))
 (segment (start 118.473858 139.610021) (end 117.4 138.536162) (width 0.5) (layer F.Cu) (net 6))
 (segment (start 161.9 138.04) (end 148.86 138.04) (width 0.5) (layer F.Cu) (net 6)))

